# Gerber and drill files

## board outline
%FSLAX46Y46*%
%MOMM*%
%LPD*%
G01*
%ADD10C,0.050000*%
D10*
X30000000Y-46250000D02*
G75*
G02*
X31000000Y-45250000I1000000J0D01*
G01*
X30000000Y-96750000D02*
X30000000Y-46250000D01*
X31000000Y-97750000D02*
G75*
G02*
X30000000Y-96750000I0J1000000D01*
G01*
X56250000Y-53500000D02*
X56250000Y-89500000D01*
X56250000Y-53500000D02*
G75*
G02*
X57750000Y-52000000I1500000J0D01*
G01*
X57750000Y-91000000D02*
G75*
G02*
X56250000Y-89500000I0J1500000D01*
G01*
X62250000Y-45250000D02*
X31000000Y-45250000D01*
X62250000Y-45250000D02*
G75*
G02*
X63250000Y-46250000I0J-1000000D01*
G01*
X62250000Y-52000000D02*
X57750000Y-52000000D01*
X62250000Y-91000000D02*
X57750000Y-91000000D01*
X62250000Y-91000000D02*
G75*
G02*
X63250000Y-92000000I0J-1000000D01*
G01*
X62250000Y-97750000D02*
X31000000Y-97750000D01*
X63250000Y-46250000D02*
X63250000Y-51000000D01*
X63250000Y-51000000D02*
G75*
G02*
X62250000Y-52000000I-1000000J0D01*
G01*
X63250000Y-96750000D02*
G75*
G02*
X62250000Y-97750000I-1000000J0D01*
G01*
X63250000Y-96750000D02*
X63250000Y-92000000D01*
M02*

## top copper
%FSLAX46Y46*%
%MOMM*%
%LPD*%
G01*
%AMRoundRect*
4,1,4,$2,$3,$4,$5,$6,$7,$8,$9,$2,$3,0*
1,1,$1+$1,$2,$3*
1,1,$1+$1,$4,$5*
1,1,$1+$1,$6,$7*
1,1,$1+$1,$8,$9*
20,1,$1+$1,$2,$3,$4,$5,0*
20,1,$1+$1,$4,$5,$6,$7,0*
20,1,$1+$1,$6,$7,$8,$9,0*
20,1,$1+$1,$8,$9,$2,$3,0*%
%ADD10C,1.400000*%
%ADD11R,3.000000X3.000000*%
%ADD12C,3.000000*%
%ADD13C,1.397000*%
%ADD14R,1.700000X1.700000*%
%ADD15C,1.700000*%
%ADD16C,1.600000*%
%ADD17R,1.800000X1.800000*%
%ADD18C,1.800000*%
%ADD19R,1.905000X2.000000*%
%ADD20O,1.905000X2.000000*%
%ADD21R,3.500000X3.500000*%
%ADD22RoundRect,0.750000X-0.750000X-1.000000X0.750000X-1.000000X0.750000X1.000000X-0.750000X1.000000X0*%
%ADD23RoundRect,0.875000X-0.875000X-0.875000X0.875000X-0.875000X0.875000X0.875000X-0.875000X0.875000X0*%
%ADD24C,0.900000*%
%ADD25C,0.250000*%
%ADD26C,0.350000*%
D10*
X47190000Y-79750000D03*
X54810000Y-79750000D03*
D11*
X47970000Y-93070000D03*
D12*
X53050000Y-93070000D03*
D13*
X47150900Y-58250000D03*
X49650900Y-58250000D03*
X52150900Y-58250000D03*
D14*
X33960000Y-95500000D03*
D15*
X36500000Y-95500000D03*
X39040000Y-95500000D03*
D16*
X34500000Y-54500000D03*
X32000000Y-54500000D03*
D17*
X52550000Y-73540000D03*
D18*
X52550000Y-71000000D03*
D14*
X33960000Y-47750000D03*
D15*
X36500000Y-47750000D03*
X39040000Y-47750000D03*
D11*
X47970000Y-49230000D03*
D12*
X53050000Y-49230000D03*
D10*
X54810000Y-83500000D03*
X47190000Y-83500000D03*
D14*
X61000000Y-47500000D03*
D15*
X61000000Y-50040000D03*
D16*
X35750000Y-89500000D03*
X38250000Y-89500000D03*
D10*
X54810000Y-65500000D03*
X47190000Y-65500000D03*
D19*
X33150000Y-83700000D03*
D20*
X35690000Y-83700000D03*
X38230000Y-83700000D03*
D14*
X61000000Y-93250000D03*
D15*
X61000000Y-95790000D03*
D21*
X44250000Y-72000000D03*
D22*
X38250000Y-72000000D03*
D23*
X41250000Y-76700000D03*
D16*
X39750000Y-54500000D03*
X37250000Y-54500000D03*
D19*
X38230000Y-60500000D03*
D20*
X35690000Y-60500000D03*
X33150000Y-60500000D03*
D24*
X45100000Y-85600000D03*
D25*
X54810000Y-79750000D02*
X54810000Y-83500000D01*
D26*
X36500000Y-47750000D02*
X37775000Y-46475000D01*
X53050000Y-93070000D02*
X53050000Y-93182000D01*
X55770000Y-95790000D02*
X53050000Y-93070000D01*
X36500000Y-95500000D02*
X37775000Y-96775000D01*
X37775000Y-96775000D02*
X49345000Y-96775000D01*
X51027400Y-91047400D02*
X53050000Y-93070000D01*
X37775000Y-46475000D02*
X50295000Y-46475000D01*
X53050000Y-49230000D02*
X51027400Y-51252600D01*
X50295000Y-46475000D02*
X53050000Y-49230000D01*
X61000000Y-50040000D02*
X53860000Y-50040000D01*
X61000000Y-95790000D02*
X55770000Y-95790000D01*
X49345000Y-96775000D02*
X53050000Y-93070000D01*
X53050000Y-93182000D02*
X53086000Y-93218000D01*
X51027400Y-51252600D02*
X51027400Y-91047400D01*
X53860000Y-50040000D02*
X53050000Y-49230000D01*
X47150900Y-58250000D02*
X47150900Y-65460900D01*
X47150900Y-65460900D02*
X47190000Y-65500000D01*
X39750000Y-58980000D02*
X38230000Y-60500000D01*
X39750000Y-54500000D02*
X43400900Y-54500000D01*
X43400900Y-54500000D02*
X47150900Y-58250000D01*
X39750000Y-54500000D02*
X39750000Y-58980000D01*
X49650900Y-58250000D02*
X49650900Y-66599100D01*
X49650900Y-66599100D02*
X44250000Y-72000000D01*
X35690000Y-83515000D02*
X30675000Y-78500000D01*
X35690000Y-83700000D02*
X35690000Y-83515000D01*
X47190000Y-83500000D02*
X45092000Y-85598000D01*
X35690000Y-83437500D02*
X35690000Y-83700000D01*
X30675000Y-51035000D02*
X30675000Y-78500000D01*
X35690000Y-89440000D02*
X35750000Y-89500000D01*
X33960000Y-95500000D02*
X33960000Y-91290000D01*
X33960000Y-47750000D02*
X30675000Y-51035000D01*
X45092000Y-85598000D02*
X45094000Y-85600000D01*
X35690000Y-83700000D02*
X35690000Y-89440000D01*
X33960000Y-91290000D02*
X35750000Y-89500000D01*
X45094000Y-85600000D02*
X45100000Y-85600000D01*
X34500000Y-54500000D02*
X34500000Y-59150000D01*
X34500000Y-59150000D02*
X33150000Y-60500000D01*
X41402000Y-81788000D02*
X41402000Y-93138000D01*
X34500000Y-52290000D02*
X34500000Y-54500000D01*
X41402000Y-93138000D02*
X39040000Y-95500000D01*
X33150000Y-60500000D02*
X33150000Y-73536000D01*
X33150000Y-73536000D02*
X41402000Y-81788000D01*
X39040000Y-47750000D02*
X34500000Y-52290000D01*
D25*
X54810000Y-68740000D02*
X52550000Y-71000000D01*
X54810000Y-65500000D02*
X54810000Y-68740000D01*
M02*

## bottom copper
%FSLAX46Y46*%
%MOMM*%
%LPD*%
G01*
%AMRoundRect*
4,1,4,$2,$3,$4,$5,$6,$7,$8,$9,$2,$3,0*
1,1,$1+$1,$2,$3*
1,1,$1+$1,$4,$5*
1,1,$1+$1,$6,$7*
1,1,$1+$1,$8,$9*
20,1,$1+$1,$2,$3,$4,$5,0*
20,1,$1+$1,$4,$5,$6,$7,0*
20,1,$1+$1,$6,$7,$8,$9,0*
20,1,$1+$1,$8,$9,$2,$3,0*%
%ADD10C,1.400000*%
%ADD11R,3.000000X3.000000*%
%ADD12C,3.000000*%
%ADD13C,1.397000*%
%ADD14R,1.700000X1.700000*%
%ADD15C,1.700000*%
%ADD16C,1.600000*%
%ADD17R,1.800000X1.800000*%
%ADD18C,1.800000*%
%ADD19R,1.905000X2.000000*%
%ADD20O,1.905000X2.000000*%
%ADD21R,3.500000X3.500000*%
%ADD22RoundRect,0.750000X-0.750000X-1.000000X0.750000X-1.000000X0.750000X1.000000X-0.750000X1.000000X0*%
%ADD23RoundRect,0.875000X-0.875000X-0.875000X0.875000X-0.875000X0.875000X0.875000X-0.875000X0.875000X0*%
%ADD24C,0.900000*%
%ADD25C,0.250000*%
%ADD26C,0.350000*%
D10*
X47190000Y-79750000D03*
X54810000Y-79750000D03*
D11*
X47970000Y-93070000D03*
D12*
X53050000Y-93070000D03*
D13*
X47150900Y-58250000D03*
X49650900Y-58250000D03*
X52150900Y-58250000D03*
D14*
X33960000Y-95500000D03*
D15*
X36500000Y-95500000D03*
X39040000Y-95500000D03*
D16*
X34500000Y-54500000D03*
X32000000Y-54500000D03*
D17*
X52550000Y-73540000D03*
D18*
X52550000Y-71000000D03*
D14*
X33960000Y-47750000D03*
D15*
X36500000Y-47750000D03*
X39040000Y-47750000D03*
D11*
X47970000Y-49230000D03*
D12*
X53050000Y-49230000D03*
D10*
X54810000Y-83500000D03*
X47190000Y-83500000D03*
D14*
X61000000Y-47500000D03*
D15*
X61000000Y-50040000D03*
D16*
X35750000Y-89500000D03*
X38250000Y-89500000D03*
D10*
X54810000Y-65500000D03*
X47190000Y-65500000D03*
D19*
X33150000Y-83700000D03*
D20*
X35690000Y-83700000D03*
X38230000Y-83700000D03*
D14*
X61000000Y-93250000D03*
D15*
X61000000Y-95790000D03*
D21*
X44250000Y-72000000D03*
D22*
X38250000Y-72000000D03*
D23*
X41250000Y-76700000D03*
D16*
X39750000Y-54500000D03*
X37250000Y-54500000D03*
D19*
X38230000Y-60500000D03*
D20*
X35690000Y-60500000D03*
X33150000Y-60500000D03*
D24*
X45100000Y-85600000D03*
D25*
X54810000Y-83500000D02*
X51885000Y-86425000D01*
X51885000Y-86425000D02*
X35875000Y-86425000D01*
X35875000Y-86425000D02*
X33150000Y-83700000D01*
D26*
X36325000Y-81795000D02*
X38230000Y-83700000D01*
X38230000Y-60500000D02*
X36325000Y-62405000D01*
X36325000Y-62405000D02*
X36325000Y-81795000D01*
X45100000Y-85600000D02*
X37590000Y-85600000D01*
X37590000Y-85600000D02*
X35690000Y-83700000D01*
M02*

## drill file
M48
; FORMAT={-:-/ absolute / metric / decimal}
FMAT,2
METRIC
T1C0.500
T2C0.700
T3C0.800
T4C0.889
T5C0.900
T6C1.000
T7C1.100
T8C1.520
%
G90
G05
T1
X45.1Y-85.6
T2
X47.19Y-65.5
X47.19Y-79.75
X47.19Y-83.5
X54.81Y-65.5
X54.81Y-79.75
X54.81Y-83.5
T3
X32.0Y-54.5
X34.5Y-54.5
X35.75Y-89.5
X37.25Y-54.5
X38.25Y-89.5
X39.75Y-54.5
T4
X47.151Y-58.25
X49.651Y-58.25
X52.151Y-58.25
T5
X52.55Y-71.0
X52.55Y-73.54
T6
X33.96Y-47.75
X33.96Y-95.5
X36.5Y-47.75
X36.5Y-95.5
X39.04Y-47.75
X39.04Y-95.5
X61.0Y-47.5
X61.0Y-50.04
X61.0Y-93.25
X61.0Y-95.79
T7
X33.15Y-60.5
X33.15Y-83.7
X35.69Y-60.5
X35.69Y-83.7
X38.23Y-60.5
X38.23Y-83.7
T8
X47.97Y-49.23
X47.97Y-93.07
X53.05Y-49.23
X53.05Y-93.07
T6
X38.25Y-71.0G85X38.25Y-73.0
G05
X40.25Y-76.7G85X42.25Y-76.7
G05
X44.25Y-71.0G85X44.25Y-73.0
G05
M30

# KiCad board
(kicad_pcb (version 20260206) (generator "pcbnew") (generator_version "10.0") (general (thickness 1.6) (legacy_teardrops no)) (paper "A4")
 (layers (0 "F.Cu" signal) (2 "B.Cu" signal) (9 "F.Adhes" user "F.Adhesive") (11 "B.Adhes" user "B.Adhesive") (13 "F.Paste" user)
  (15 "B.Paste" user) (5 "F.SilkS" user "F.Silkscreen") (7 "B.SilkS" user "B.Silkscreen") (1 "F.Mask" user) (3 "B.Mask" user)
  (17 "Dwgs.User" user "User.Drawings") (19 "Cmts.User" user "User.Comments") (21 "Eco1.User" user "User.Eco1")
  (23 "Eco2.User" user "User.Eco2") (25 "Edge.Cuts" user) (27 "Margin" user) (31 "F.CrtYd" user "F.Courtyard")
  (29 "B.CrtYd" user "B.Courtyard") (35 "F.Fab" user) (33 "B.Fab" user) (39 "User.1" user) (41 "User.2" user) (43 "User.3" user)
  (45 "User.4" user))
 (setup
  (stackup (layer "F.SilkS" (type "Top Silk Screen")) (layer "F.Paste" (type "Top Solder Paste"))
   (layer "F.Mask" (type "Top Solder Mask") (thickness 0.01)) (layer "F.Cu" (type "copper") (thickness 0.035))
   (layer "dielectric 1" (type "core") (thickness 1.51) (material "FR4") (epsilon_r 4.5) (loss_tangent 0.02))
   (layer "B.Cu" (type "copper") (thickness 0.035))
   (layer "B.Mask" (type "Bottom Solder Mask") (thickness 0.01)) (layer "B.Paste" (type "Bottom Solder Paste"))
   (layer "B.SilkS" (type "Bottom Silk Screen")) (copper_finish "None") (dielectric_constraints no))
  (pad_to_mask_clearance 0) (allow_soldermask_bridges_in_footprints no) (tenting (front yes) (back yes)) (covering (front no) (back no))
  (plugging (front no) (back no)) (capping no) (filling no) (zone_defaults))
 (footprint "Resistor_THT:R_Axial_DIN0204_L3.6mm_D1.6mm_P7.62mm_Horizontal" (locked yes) (layer "F.Cu") (at 47.19 79.75)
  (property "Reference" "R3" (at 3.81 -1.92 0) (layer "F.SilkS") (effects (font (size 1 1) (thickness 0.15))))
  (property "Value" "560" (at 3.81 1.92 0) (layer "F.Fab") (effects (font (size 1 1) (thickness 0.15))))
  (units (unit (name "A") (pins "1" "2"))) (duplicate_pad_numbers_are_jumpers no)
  (pad "1" thru_hole circle (at 0 0) (size 1.4 1.4) (drill 0.7) (layers "*.Cu" "*.Mask") (remove_unused_layers no) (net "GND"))
  (pad "2" thru_hole circle (at 7.62 0) (size 1.4 1.4) (drill 0.7) (layers "*.Cu" "*.Mask") (remove_unused_layers no) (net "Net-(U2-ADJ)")))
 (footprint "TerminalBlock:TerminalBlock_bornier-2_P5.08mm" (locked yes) (layer "F.Cu") (at 47.97 93.07)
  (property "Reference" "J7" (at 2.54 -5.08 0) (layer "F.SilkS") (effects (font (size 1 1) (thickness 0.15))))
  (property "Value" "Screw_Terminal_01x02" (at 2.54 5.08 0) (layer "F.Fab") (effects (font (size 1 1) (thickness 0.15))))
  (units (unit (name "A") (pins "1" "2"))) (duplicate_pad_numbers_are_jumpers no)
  (pad "1" thru_hole rect (at 0 0) (size 3 3) (drill 1.52) (layers "*.Cu" "*.Mask") (remove_unused_layers no) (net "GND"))
  (pad "2" thru_hole circle (at 5.08 0) (size 3 3) (drill 1.52) (layers "*.Cu" "*.Mask") (remove_unused_layers no) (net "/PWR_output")))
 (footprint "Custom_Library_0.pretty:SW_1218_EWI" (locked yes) (layer "F.Cu") (at 47.1509 58.25 90)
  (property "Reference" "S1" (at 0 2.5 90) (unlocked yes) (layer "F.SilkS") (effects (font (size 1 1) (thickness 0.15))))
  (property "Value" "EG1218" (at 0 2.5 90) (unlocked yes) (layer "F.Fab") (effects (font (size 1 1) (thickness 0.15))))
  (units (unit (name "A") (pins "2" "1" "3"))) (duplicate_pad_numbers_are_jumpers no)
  (pad "1" thru_hole circle (at 0 0 90) (size 1.397 1.397) (drill 0.889) (layers "*.Cu" "*.Mask") (remove_unused_layers no) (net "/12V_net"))
  (pad "2" thru_hole circle (at 0 2.5 90) (size 1.397 1.397) (drill 0.889) (layers "*.Cu" "*.Mask") (remove_unused_layers no)
   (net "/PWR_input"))
  (pad "3" thru_hole circle (at 0 5 90) (size 1.397 1.397) (drill 0.889) (layers "*.Cu" "*.Mask") (remove_unused_layers no)
   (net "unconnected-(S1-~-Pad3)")))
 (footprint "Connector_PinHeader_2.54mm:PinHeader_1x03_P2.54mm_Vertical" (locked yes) (layer "F.Cu") (at 33.96 95.5 90)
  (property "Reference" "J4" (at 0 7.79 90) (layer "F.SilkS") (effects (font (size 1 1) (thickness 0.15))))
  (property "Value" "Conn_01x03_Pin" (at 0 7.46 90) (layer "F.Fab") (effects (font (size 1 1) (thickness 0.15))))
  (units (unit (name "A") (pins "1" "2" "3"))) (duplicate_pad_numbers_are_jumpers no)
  (pad "1" thru_hole rect (at 0 0 90) (size 1.7 1.7) (drill 1) (layers "*.Cu" "*.Mask") (remove_unused_layers no) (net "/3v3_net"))
  (pad "2" thru_hole circle (at 0 2.54 90) (size 1.7 1.7) (drill 1) (layers "*.Cu" "*.Mask") (remove_unused_layers no) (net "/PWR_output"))
  (pad "3" thru_hole circle (at 0 5.08 90) (size 1.7 1.7) (drill 1) (layers "*.Cu" "*.Mask") (remove_unused_layers no) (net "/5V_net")))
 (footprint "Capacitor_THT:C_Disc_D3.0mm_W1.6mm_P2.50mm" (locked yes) (layer "F.Cu") (at 34.5 54.5 180)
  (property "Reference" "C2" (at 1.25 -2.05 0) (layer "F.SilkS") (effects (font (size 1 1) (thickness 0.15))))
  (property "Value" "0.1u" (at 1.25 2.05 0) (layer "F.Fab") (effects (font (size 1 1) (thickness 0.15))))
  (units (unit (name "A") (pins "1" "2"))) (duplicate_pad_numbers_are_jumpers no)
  (pad "1" thru_hole circle (at 0 0 180) (size 1.6 1.6) (drill 0.8) (layers "*.Cu" "*.Mask") (remove_unused_layers no) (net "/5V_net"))
  (pad "2" thru_hole circle (at 2.5 0 180) (size 1.6 1.6) (drill 0.8) (layers "*.Cu" "*.Mask") (remove_unused_layers no) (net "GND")))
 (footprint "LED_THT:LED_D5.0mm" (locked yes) (layer "F.Cu") (at 52.55 73.54 90)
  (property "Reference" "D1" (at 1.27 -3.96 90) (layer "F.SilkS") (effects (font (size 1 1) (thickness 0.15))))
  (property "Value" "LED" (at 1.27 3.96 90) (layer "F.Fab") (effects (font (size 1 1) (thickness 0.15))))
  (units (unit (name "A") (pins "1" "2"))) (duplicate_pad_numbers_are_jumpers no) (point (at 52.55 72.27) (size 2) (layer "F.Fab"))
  (pad "1" thru_hole rect (at 0 0 90) (size 1.8 1.8) (drill 0.9) (layers "*.Cu" "*.Mask") (remove_unused_layers no) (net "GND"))
  (pad "2" thru_hole circle (at 2.54 0 90) (size 1.8 1.8) (drill 0.9) (layers "*.Cu" "*.Mask") (remove_unused_layers no) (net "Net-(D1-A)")))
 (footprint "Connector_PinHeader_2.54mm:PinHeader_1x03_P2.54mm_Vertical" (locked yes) (layer "F.Cu") (at 33.96 47.75 90)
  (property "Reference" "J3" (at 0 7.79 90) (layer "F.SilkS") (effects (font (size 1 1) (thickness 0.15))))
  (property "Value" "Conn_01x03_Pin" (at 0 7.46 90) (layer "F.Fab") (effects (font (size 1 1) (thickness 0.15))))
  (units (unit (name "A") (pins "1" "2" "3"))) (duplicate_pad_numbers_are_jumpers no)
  (pad "1" thru_hole rect (at 0 0 90) (size 1.7 1.7) (drill 1) (layers "*.Cu" "*.Mask") (remove_unused_layers no) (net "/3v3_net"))
  (pad "2" thru_hole circle (at 0 2.54 90) (size 1.7 1.7) (drill 1) (layers "*.Cu" "*.Mask") (remove_unused_layers no) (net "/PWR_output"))
  (pad "3" thru_hole circle (at 0 5.08 90) (size 1.7 1.7) (drill 1) (layers "*.Cu" "*.Mask") (remove_unused_layers no) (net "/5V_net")))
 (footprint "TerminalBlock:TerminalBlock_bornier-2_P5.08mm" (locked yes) (layer "F.Cu") (at 47.97 49.23)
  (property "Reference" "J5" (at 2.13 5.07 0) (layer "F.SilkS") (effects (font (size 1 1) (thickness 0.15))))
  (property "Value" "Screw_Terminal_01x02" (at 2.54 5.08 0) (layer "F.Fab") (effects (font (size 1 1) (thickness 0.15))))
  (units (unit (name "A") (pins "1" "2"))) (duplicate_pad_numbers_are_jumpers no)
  (pad "1" thru_hole rect (at 0 0) (size 3 3) (drill 1.52) (layers "*.Cu" "*.Mask") (remove_unused_layers no) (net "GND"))
  (pad "2" thru_hole circle (at 5.08 0) (size 3 3) (drill 1.52) (layers "*.Cu" "*.Mask") (remove_unused_layers no) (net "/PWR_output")))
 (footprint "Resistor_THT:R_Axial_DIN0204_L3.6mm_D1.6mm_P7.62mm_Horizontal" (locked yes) (layer "F.Cu") (at 54.81 83.5 180)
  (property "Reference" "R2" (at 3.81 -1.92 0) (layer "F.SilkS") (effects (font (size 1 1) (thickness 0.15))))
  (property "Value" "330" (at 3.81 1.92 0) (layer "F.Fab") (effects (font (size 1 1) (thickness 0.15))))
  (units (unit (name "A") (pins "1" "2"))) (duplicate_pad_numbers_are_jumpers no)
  (pad "1" thru_hole circle (at 0 0 180) (size 1.4 1.4) (drill 0.7) (layers "*.Cu" "*.Mask") (remove_unused_layers no) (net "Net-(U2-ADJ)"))
  (pad "2" thru_hole circle (at 7.62 0 180) (size 1.4 1.4) (drill 0.7) (layers "*.Cu" "*.Mask") (remove_unused_layers no) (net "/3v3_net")))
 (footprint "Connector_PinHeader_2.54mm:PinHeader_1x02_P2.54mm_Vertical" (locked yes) (layer "F.Cu") (at 61 47.5)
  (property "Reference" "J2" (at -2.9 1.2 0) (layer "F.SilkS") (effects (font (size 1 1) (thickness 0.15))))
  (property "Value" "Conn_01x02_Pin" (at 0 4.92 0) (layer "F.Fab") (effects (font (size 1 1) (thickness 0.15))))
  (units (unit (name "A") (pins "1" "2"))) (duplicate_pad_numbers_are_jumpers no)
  (pad "1" thru_hole rect (at 0 0) (size 1.7 1.7) (drill 1) (layers "*.Cu" "*.Mask") (remove_unused_layers no) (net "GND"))
  (pad "2" thru_hole circle (at 0 2.54) (size 1.7 1.7) (drill 1) (layers "*.Cu" "*.Mask") (remove_unused_layers no) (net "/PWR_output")))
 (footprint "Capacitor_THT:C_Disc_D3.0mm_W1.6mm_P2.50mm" (layer "F.Cu") (at 35.75 89.5)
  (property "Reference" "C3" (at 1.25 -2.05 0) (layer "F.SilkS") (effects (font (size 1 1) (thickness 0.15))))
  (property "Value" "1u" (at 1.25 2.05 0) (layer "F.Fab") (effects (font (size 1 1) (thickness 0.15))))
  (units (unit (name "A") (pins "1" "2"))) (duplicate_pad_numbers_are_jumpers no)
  (pad "1" thru_hole circle (at 0 0) (size 1.6 1.6) (drill 0.8) (layers "*.Cu" "*.Mask") (remove_unused_layers no) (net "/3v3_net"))
  (pad "2" thru_hole circle (at 2.5 0) (size 1.6 1.6) (drill 0.8) (layers "*.Cu" "*.Mask") (remove_unused_layers no) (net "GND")))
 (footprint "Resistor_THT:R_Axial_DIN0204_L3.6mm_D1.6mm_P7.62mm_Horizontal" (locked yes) (layer "F.Cu") (at 54.81 65.5 180)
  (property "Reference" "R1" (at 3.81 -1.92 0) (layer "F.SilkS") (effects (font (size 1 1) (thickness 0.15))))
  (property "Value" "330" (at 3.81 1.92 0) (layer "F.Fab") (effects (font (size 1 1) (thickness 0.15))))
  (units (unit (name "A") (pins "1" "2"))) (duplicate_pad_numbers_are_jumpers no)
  (pad "1" thru_hole circle (at 0 0 180) (size 1.4 1.4) (drill 0.7) (layers "*.Cu" "*.Mask") (remove_unused_layers no) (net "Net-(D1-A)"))
  (pad "2" thru_hole circle (at 7.62 0 180) (size 1.4 1.4) (drill 0.7) (layers "*.Cu" "*.Mask") (remove_unused_layers no) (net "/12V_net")))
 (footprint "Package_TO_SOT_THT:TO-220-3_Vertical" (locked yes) (layer "F.Cu") (at 33.15 83.7)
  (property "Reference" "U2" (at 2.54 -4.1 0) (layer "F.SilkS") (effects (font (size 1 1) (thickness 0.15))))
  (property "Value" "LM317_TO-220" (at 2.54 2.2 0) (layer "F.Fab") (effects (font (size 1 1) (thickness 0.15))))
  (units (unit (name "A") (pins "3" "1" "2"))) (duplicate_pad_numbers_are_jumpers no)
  (pad "1" thru_hole rect (at 0 0) (size 1.905 2) (drill 1.1) (layers "*.Cu" "*.Mask") (remove_unused_layers no) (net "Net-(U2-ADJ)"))
  (pad "2" thru_hole oval (at 2.54 0) (size 1.905 2) (drill 1.1) (layers "*.Cu" "*.Mask") (remove_unused_layers no) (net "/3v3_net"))
  (pad "3" thru_hole oval (at 5.08 0) (size 1.905 2) (drill 1.1) (layers "*.Cu" "*.Mask") (remove_unused_layers no) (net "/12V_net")))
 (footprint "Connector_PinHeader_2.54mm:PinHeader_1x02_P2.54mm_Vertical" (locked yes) (layer "F.Cu") (at 61 93.25)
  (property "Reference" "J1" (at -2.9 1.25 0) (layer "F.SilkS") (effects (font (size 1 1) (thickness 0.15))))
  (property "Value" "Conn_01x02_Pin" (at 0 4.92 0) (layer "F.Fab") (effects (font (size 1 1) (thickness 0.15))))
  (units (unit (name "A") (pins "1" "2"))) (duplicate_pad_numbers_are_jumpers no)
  (pad "1" thru_hole rect (at 0 0) (size 1.7 1.7) (drill 1) (layers "*.Cu" "*.Mask") (remove_unused_layers no) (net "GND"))
  (pad "2" thru_hole circle (at 0 2.54) (size 1.7 1.7) (drill 1) (layers "*.Cu" "*.Mask") (remove_unused_layers no) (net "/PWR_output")))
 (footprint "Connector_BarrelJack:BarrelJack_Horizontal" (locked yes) (layer "F.Cu") (at 44.25 72)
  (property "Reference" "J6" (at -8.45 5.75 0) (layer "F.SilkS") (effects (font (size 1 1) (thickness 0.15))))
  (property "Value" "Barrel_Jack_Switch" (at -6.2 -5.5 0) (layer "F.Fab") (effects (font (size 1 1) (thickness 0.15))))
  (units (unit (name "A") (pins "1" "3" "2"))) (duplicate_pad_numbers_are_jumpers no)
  (pad "1" thru_hole rect (at 0 0) (size 3.5 3.5) (drill oval 1 3) (layers "*.Cu" "*.Mask") (remove_unused_layers no) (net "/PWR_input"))
  (pad "2" thru_hole roundrect (at -6 0) (size 3 3.5) (drill oval 1 3) (layers "*.Cu" "*.Mask") (remove_unused_layers no)
   (roundrect_rratio 0.25) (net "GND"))
  (pad "3" thru_hole roundrect (at -3 4.7) (size 3.5 3.5) (drill oval 3 1) (layers "*.Cu" "*.Mask") (remove_unused_layers no)
   (roundrect_rratio 0.25) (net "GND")))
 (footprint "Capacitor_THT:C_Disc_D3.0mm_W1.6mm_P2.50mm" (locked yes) (layer "F.Cu") (at 39.75 54.5 180)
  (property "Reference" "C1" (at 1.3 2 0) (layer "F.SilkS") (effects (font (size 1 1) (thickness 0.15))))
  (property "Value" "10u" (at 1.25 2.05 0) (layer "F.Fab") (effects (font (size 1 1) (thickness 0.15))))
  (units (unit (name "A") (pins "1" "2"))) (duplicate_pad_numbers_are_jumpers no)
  (pad "1" thru_hole circle (at 0 0 180) (size 1.6 1.6) (drill 0.8) (layers "*.Cu" "*.Mask") (remove_unused_layers no) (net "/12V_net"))
  (pad "2" thru_hole circle (at 2.5 0 180) (size 1.6 1.6) (drill 0.8) (layers "*.Cu" "*.Mask") (remove_unused_layers no) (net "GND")))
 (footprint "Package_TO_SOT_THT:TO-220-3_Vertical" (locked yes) (layer "F.Cu") (at 38.23 60.5 180)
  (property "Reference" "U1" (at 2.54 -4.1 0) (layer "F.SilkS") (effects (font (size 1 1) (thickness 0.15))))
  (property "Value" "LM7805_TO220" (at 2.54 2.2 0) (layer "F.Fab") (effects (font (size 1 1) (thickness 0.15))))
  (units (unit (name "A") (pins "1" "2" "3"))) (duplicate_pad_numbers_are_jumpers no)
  (pad "1" thru_hole rect (at 0 0 180) (size 1.905 2) (drill 1.1) (layers "*.Cu" "*.Mask") (remove_unused_layers no) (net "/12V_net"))
  (pad "2" thru_hole oval (at 2.54 0 180) (size 1.905 2) (drill 1.1) (layers "*.Cu" "*.Mask") (remove_unused_layers no) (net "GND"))
  (pad "3" thru_hole oval (at 5.08 0 180) (size 1.905 2) (drill 1.1) (layers "*.Cu" "*.Mask") (remove_unused_layers no) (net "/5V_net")))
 (gr_arc (start 30 46.25) (mid 30.292893 45.542893) (end 31 45.25) (stroke (width 0.05) (type default)) (layer "Edge.Cuts"))
 (gr_line (start 30 96.75) (end 30 46.25) (stroke (width 0.05) (type default)) (layer "Edge.Cuts"))
 (gr_arc (start 31 97.75) (mid 30.292893 97.457107) (end 30 96.75) (stroke (width 0.05) (type default)) (layer "Edge.Cuts"))
 (gr_line (start 56.25 53.5) (end 56.25 89.5) (stroke (width 0.05) (type default)) (layer "Edge.Cuts"))
 (gr_arc (start 56.25 53.5) (mid 56.68934 52.43934) (end 57.75 52) (stroke (width 0.05) (type default)) (layer "Edge.Cuts"))
 (gr_arc (start 57.75 91) (mid 56.68934 90.56066) (end 56.25 89.5) (stroke (width 0.05) (type default)) (layer "Edge.Cuts"))
 (gr_line (start 62.25 45.25) (end 31 45.25) (stroke (width 0.05) (type default)) (layer "Edge.Cuts"))
 (gr_arc (start 62.25 45.25) (mid 62.957107 45.542893) (end 63.25 46.25) (stroke (width 0.05) (type default)) (layer "Edge.Cuts"))
 (gr_line (start 62.25 52) (end 57.75 52) (stroke (width 0.05) (type default)) (layer "Edge.Cuts"))
 (gr_line (start 62.25 91) (end 57.75 91) (stroke (width 0.05) (type default)) (layer "Edge.Cuts"))
 (gr_arc (start 62.25 91) (mid 62.957107 91.292893) (end 63.25 92) (stroke (width 0.05) (type default)) (layer "Edge.Cuts"))
 (gr_line (start 62.25 97.75) (end 31 97.75) (stroke (width 0.05) (type default)) (layer "Edge.Cuts"))
 (gr_line (start 63.25 46.25) (end 63.25 51) (stroke (width 0.05) (type default)) (layer "Edge.Cuts"))
 (gr_arc (start 63.25 51) (mid 62.957107 51.707107) (end 62.25 52) (stroke (width 0.05) (type default)) (layer "Edge.Cuts"))
 (gr_arc (start 63.25 96.75) (mid 62.957107 97.457107) (end 62.25 97.75) (stroke (width 0.05) (type default)) (layer "Edge.Cuts"))
 (gr_line (start 63.25 96.75) (end 63.25 92) (stroke (width 0.05) (type default)) (layer "Edge.Cuts"))
 (segment (start 54.81 79.75) (end 54.81 83.5) (width 0.25) (layer "F.Cu") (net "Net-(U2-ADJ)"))
 (segment (start 54.81 83.5) (end 51.885 86.425) (width 0.25) (layer "B.Cu") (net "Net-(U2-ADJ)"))
 (segment (start 51.885 86.425) (end 35.875 86.425) (width 0.25) (layer "B.Cu") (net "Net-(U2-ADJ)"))
 (segment (start 35.875 86.425) (end 33.15 83.7) (width 0.25) (layer "B.Cu") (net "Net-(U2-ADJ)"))
 (segment (start 36.5 47.75) (end 37.775 46.475) (width 0.35) (layer "F.Cu") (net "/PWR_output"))
 (segment (start 53.05 93.07) (end 53.05 93.182) (width 0.35) (layer "F.Cu") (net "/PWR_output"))
 (segment (start 55.77 95.79) (end 53.05 93.07) (width 0.35) (layer "F.Cu") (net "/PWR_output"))
 (segment (start 36.5 95.5) (end 37.775 96.775) (width 0.35) (layer "F.Cu") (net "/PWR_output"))
 (segment (start 37.775 96.775) (end 49.345 96.775) (width 0.35) (layer "F.Cu") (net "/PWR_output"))
 (segment (start 51.0274 91.0474) (end 53.05 93.07) (width 0.35) (layer "F.Cu") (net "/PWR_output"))
 (segment (start 37.775 46.475) (end 50.295 46.475) (width 0.35) (layer "F.Cu") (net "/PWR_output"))
 (segment (start 53.05 49.23) (end 51.0274 51.2526) (width 0.35) (layer "F.Cu") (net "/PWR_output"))
 (segment (start 50.295 46.475) (end 53.05 49.23) (width 0.35) (layer "F.Cu") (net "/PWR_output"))
 (segment (start 61 50.04) (end 53.86 50.04) (width 0.35) (layer "F.Cu") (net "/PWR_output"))
 (segment (start 61 95.79) (end 55.77 95.79) (width 0.35) (layer "F.Cu") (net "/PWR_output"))
 (segment (start 49.345 96.775) (end 53.05 93.07) (width 0.35) (layer "F.Cu") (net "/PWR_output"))
 (segment (start 53.05 93.182) (end 53.086 93.218) (width 0.35) (layer "F.Cu") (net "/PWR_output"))
 (segment (start 51.0274 51.2526) (end 51.0274 91.0474) (width 0.35) (layer "F.Cu") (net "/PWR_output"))
 (segment (start 53.86 50.04) (end 53.05 49.23) (width 0.35) (layer "F.Cu") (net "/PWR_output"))
 (segment (start 47.1509 58.25) (end 47.1509 65.4609) (width 0.35) (layer "F.Cu") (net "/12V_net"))
 (segment (start 47.1509 65.4609) (end 47.19 65.5) (width 0.35) (layer "F.Cu") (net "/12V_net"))
 (segment (start 39.75 58.98) (end 38.23 60.5) (width 0.35) (layer "F.Cu") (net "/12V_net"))
 (segment (start 39.75 54.5) (end 43.4009 54.5) (width 0.35) (layer "F.Cu") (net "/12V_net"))
 (segment (start 43.4009 54.5) (end 47.1509 58.25) (width 0.35) (layer "F.Cu") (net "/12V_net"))
 (segment (start 39.75 54.5) (end 39.75 58.98) (width 0.35) (layer "F.Cu") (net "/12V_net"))
 (segment (start 36.325 81.795) (end 38.23 83.7) (width 0.35) (layer "B.Cu") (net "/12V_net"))
 (segment (start 38.23 60.5) (end 36.325 62.405) (width 0.35) (layer "B.Cu") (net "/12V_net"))
 (segment (start 36.325 62.405) (end 36.325 81.795) (width 0.35) (layer "B.Cu") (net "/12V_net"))
 (segment (start 49.6509 58.25) (end 49.6509 66.5991) (width 0.35) (layer "F.Cu") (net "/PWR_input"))
 (segment (start 49.6509 66.5991) (end 44.25 72) (width 0.35) (layer "F.Cu") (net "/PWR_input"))
 (segment (start 35.69 83.515) (end 30.675 78.5) (width 0.35) (layer "F.Cu") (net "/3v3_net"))
 (segment (start 35.69 83.7) (end 35.69 83.515) (width 0.35) (layer "F.Cu") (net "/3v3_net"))
 (segment (start 47.19 83.5) (end 45.092 85.598) (width 0.35) (layer "F.Cu") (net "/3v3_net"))
 (segment (start 35.69 83.4375) (end 35.69 83.7) (width 0.35) (layer "F.Cu") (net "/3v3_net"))
 (segment (start 30.675 51.035) (end 30.675 78.5) (width 0.35) (layer "F.Cu") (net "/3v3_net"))
 (segment (start 35.69 89.44) (end 35.75 89.5) (width 0.35) (layer "F.Cu") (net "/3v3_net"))
 (segment (start 33.96 95.5) (end 33.96 91.29) (width 0.35) (layer "F.Cu") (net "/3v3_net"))
 (segment (start 33.96 47.75) (end 30.675 51.035) (width 0.35) (layer "F.Cu") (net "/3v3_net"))
 (segment (start 45.092 85.598) (end 45.094 85.6) (width 0.35) (layer "F.Cu") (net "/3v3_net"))
 (segment (start 35.69 83.7) (end 35.69 89.44) (width 0.35) (layer "F.Cu") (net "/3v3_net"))
 (segment (start 33.96 91.29) (end 35.75 89.5) (width 0.35) (layer "F.Cu") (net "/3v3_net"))
 (segment (start 45.094 85.6) (end 45.1 85.6) (width 0.35) (layer "F.Cu") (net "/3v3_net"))
 (via (at 45.1 85.6) (size 0.9) (drill 0.5) (layers "F.Cu" "B.Cu") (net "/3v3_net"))
 (segment (start 45.1 85.6) (end 37.59 85.6) (width 0.35) (layer "B.Cu") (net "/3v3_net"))
 (segment (start 37.59 85.6) (end 35.69 83.7) (width 0.35) (layer "B.Cu") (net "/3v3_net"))
 (segment (start 34.5 54.5) (end 34.5 59.15) (width 0.35) (layer "F.Cu") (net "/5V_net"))
 (segment (start 34.5 59.15) (end 33.15 60.5) (width 0.35) (layer "F.Cu") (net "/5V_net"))
 (segment (start 41.402 81.788) (end 41.402 93.138) (width 0.35) (layer "F.Cu") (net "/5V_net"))
 (segment (start 34.5 52.29) (end 34.5 54.5) (width 0.35) (layer "F.Cu") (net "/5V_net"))
 (segment (start 41.402 93.138) (end 39.04 95.5) (width 0.35) (layer "F.Cu") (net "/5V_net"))
 (segment (start 33.15 60.5) (end 33.15 73.536) (width 0.35) (layer "F.Cu") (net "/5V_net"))
 (segment (start 33.15 73.536) (end 41.402 81.788) (width 0.35) (layer "F.Cu") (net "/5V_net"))
 (segment (start 39.04 47.75) (end 34.5 52.29) (width 0.35) (layer "F.Cu") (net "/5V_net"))
 (segment (start 54.81 68.74) (end 52.55 71) (width 0.25) (layer "F.Cu") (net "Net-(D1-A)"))
 (segment (start 54.81 65.5) (end 54.81 68.74) (width 0.25) (layer "F.Cu") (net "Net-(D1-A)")))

